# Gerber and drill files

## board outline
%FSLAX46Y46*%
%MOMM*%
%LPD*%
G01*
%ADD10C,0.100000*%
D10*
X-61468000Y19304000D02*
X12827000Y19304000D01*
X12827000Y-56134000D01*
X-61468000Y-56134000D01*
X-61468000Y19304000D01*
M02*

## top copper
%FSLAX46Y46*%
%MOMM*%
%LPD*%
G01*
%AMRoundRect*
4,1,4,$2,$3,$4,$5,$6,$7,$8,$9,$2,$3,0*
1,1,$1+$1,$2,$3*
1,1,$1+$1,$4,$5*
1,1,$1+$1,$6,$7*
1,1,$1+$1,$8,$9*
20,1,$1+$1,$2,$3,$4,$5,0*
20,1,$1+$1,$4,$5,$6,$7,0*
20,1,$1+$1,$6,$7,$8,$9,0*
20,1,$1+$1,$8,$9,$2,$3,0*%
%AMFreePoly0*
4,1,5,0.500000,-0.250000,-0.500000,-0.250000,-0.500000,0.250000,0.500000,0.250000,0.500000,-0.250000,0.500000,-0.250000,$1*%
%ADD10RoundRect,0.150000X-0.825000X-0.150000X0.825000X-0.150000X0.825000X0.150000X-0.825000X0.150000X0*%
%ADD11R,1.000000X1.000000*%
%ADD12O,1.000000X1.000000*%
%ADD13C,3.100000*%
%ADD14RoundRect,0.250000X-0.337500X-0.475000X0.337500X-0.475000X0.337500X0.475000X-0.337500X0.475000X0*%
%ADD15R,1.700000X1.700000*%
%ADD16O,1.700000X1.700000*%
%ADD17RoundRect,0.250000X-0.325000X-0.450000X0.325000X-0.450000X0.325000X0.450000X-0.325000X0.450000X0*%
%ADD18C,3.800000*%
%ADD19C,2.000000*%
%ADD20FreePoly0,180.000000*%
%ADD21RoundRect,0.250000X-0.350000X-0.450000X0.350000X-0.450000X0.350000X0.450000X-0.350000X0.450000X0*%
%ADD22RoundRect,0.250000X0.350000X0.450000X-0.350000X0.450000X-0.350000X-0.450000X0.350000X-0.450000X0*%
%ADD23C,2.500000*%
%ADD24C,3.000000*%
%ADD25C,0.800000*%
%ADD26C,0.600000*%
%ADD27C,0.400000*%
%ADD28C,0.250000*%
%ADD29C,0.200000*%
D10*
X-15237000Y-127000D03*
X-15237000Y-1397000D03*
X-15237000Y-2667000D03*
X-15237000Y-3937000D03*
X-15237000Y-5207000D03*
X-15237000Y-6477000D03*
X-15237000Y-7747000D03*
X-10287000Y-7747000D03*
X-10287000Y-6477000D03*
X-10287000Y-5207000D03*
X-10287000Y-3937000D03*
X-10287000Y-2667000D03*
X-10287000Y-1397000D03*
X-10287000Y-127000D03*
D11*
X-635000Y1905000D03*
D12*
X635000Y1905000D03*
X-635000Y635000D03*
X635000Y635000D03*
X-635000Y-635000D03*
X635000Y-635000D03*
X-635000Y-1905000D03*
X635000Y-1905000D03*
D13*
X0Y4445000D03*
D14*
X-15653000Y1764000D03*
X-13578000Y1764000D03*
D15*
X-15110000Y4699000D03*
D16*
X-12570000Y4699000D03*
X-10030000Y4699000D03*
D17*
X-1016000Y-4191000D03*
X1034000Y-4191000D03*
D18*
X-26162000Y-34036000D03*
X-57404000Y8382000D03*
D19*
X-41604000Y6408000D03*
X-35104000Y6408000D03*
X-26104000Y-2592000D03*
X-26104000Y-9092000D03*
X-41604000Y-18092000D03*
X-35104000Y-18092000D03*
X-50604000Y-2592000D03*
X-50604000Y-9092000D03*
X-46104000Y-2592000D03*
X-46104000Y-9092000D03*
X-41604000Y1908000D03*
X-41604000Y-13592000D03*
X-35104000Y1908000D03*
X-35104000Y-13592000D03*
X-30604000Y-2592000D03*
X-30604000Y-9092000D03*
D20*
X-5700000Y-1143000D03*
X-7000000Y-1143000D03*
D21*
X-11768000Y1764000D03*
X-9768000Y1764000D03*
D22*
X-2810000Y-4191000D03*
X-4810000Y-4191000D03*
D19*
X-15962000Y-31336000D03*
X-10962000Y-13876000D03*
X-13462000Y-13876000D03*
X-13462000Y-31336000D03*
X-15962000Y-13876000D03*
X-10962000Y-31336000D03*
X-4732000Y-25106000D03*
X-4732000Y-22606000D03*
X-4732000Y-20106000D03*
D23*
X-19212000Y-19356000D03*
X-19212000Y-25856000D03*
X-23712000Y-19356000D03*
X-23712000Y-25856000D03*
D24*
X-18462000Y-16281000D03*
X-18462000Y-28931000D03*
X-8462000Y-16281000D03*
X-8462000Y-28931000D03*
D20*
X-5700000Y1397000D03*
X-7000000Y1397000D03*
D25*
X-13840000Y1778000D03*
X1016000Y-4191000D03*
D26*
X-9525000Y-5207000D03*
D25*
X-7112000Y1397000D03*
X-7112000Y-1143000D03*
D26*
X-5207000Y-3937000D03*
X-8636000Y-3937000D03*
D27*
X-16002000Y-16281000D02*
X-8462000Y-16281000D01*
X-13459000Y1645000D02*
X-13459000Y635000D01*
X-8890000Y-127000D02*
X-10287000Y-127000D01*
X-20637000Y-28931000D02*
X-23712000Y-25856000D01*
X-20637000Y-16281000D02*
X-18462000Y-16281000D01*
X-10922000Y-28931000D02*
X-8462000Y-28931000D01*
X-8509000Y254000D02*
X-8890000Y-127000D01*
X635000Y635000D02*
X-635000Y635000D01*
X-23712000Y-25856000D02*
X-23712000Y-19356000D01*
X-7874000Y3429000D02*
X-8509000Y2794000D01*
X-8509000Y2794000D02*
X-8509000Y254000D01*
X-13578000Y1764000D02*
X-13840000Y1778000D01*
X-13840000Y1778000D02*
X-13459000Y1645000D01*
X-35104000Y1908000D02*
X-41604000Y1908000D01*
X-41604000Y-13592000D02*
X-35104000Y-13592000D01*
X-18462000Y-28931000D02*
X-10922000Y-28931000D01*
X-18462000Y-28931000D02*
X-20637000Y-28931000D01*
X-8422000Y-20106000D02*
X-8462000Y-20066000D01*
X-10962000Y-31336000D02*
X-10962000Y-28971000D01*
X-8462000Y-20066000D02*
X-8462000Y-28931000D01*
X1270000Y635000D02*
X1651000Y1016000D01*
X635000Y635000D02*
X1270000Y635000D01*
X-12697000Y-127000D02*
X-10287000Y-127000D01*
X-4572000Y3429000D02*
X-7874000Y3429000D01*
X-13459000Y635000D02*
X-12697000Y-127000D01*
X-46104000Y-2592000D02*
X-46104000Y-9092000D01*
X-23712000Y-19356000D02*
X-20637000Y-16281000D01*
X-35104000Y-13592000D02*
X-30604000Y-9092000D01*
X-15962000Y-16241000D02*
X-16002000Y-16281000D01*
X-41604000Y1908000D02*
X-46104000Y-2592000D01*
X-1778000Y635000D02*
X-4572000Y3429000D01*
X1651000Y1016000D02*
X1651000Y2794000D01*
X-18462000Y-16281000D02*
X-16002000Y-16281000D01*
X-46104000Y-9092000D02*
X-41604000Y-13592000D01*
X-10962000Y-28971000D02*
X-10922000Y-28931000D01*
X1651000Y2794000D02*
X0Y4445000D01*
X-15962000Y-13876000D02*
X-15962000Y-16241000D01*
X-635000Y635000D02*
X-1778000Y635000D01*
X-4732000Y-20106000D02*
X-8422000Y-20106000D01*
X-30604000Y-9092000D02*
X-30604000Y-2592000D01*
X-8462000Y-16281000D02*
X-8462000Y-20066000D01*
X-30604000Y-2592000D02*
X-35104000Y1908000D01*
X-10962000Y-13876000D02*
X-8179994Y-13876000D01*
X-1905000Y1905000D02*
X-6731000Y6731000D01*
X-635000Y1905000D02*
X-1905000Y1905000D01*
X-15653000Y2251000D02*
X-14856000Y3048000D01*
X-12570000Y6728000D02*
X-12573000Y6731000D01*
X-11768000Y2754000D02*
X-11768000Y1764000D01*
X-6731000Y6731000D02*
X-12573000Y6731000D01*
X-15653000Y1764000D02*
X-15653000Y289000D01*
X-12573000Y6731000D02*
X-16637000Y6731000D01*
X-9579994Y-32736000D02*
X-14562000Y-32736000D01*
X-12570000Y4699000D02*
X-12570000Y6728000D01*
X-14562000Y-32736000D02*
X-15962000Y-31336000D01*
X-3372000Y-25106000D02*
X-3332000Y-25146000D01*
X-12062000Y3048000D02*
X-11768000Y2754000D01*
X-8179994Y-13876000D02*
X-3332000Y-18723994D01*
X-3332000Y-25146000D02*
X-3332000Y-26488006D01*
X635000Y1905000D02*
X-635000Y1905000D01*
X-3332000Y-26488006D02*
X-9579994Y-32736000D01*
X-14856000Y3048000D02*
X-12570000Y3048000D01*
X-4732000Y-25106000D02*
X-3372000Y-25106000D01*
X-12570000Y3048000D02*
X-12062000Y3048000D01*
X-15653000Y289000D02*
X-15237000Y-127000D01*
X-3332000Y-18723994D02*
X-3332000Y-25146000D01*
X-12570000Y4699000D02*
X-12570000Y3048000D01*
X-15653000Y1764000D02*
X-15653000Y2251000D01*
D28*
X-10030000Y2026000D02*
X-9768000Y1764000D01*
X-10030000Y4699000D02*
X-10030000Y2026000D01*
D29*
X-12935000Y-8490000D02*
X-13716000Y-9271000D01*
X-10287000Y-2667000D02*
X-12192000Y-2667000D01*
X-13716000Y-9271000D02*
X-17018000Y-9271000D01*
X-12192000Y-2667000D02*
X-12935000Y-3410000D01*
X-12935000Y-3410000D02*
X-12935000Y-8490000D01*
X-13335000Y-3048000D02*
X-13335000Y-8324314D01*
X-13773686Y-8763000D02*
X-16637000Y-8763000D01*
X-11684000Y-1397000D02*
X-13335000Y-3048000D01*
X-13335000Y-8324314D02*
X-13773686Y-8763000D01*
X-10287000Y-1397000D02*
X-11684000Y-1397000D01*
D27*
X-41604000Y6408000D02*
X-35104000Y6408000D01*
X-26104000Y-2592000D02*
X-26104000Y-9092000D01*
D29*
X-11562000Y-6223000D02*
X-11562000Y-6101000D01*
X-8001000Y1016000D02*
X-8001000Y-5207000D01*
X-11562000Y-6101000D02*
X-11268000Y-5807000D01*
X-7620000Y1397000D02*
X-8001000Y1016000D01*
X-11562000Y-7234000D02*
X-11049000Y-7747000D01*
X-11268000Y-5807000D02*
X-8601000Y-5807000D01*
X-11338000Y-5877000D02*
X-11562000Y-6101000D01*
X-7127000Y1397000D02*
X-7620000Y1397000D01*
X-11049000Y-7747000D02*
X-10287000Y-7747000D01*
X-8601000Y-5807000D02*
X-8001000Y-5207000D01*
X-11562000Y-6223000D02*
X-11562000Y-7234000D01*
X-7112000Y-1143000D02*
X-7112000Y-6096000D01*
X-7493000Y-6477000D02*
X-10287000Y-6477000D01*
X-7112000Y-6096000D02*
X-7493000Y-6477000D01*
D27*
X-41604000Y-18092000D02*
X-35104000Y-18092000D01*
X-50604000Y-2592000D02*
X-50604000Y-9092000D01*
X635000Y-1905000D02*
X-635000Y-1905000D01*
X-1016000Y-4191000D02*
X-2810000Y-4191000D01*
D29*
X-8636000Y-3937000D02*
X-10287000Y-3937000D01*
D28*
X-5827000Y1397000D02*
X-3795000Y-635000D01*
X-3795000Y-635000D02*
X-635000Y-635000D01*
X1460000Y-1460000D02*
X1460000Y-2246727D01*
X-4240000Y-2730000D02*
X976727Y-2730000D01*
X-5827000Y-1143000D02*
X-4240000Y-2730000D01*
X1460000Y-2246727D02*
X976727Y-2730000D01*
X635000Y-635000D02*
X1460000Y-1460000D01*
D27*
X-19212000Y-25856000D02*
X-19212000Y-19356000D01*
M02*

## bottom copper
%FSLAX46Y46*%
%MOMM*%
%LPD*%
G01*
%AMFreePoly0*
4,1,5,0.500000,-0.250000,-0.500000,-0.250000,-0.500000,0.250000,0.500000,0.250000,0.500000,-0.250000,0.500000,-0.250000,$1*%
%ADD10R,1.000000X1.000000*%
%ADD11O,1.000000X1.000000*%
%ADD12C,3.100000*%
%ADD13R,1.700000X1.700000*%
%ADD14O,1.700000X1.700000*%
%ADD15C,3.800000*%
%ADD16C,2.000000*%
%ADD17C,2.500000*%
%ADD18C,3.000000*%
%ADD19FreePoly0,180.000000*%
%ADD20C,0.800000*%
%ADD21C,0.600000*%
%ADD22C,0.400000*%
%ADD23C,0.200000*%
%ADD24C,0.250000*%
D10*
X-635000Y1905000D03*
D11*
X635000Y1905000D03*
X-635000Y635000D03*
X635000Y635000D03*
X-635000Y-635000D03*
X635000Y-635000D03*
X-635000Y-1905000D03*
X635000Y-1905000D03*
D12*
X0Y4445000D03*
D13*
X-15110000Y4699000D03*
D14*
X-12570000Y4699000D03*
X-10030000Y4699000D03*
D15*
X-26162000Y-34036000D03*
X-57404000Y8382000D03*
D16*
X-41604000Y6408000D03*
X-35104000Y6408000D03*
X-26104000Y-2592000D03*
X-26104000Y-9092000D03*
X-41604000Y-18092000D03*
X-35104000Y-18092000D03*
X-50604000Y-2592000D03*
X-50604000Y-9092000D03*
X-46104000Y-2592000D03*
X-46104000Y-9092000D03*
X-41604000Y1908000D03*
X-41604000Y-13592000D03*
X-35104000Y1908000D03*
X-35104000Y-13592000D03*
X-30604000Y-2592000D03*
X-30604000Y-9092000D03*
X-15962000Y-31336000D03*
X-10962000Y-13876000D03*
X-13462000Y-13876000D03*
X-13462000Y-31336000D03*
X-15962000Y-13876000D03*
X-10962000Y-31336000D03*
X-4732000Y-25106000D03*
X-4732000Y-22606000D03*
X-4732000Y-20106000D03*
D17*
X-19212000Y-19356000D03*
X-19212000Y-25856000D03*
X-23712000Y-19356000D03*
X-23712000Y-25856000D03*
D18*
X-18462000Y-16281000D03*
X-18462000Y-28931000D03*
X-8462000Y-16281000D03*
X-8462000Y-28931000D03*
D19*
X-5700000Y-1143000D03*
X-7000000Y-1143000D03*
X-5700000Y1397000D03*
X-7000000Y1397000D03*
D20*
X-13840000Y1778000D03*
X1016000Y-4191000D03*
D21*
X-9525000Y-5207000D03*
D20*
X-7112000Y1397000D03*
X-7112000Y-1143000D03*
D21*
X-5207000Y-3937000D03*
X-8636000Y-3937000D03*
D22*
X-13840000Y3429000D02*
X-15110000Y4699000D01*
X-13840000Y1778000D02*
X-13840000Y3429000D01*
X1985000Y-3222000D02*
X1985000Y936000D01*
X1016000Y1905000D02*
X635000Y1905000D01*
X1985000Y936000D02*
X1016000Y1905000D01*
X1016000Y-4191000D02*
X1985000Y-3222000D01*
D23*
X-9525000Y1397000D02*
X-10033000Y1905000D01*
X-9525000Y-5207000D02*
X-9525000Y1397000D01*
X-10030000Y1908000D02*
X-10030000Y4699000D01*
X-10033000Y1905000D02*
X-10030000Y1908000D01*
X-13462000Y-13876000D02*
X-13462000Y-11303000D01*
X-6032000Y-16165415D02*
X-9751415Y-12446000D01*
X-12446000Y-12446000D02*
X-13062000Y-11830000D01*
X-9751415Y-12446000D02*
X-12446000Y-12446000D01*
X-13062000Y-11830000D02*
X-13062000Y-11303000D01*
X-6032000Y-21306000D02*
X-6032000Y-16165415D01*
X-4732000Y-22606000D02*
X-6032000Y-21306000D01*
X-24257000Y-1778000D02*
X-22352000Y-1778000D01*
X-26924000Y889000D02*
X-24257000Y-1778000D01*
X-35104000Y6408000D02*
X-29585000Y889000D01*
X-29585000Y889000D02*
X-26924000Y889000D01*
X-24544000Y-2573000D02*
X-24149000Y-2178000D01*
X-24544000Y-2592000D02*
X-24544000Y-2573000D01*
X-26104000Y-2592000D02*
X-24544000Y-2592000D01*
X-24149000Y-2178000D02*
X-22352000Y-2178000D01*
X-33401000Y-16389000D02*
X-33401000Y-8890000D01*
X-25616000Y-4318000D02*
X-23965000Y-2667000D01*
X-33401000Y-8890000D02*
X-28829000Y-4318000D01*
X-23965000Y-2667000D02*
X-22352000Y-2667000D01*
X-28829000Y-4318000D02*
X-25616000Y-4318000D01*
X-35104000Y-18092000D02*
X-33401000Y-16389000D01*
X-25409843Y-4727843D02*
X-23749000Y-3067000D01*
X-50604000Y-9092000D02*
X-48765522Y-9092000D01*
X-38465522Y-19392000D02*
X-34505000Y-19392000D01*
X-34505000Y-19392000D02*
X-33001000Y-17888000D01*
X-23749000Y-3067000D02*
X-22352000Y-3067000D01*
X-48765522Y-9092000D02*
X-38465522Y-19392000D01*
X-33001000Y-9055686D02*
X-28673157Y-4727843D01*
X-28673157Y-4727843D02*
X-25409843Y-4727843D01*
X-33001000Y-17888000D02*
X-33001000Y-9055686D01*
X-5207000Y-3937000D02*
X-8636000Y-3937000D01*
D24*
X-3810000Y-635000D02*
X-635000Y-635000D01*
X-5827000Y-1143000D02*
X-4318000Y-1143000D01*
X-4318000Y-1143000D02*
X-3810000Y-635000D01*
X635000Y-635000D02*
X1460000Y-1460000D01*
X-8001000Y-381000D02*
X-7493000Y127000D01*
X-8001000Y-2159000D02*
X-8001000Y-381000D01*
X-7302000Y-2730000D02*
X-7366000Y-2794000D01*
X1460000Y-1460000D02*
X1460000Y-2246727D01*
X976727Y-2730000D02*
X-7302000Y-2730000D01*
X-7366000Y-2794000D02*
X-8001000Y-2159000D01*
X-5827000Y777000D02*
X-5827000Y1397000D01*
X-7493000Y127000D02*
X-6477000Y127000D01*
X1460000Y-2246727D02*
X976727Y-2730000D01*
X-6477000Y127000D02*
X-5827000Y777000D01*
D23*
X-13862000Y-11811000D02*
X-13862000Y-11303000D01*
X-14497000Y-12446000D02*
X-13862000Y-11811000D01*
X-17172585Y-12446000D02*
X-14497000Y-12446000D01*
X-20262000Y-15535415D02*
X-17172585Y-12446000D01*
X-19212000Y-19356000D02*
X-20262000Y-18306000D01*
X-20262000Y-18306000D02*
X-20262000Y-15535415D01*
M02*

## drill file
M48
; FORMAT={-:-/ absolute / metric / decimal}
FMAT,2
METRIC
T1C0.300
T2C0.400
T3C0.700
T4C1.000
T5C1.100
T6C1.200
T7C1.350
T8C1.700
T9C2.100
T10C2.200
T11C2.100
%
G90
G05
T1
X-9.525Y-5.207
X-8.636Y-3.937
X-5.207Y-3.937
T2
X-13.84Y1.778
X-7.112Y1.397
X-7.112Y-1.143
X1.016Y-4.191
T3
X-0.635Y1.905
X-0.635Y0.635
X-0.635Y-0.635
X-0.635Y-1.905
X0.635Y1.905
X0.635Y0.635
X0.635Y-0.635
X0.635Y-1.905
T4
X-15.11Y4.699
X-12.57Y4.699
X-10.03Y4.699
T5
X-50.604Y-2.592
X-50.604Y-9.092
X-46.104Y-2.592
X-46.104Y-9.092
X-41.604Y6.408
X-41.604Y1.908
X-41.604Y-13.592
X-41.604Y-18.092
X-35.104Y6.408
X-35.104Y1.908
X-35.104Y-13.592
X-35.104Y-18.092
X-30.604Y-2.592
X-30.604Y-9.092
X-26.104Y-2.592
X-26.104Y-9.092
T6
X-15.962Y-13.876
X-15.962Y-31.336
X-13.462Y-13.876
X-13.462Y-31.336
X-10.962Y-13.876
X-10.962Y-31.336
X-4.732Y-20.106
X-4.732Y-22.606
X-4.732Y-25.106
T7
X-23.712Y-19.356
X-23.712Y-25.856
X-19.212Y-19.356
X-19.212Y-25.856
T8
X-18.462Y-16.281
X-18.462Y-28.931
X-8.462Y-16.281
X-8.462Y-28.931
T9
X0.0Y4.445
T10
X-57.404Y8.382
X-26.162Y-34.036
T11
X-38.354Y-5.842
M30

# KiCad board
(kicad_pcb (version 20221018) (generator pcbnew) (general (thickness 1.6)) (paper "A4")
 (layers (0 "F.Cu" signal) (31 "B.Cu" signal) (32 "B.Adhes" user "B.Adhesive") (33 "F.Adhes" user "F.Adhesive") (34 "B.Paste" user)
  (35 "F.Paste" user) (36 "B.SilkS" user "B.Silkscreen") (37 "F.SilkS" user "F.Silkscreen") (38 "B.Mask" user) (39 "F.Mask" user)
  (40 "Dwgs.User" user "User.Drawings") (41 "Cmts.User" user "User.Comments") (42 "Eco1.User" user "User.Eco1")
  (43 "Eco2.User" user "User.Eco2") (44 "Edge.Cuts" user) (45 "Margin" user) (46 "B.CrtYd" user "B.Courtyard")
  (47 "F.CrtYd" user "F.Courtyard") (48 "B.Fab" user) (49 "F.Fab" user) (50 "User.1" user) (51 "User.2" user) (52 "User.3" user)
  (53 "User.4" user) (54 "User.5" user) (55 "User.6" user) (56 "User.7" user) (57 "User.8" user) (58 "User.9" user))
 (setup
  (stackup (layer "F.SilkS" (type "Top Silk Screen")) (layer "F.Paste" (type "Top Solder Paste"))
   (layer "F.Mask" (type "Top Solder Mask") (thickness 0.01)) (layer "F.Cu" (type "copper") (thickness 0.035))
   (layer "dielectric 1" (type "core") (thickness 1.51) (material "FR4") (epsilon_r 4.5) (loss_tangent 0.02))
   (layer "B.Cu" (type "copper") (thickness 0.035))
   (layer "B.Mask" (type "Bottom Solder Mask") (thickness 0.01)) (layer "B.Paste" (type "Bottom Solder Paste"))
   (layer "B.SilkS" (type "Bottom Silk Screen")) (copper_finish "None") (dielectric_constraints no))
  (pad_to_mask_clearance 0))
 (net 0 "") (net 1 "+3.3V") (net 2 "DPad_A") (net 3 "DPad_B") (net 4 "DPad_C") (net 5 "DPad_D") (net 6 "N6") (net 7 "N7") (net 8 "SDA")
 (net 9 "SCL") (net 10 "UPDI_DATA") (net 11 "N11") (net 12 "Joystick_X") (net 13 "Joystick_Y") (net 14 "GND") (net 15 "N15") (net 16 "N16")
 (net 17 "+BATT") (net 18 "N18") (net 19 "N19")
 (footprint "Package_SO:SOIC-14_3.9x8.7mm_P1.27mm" (layer "F.Cu") (at -12.762 3.937)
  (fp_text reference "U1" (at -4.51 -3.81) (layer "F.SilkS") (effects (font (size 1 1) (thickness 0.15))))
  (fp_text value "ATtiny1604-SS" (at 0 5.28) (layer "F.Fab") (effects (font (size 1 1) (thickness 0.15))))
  (pad "1" smd roundrect (at -2.475 -3.81) (size 1.95 0.6) (layers "F.Cu" "F.Paste" "F.Mask") (roundrect_rratio 0.25) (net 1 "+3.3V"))
  (pad "2" smd roundrect (at -2.475 -2.54) (size 1.95 0.6) (layers "F.Cu" "F.Paste" "F.Mask") (roundrect_rratio 0.25) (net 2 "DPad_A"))
  (pad "3" smd roundrect (at -2.475 -1.27) (size 1.95 0.6) (layers "F.Cu" "F.Paste" "F.Mask") (roundrect_rratio 0.25) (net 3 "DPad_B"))
  (pad "4" smd roundrect (at -2.475 0) (size 1.95 0.6) (layers "F.Cu" "F.Paste" "F.Mask") (roundrect_rratio 0.25) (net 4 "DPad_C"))
  (pad "5" smd roundrect (at -2.475 1.27) (size 1.95 0.6) (layers "F.Cu" "F.Paste" "F.Mask") (roundrect_rratio 0.25) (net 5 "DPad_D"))
  (pad "6" smd roundrect (at -2.475 2.54) (size 1.95 0.6) (layers "F.Cu" "F.Paste" "F.Mask") (roundrect_rratio 0.25) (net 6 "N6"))
  (pad "7" smd roundrect (at -2.475 3.81) (size 1.95 0.6) (layers "F.Cu" "F.Paste" "F.Mask") (roundrect_rratio 0.25) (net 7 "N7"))
  (pad "8" smd roundrect (at 2.475 3.81) (size 1.95 0.6) (layers "F.Cu" "F.Paste" "F.Mask") (roundrect_rratio 0.25) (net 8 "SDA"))
  (pad "9" smd roundrect (at 2.475 2.54) (size 1.95 0.6) (layers "F.Cu" "F.Paste" "F.Mask") (roundrect_rratio 0.25) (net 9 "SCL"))
  (pad "10" smd roundrect (at 2.475 1.27) (size 1.95 0.6) (layers "F.Cu" "F.Paste" "F.Mask") (roundrect_rratio 0.25) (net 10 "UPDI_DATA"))
  (pad "11" smd roundrect (at 2.475 0) (size 1.95 0.6) (layers "F.Cu" "F.Paste" "F.Mask") (roundrect_rratio 0.25) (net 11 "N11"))
  (pad "12" smd roundrect (at 2.475 -1.27) (size 1.95 0.6) (layers "F.Cu" "F.Paste" "F.Mask") (roundrect_rratio 0.25) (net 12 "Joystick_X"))
  (pad "13" smd roundrect (at 2.475 -2.54) (size 1.95 0.6) (layers "F.Cu" "F.Paste" "F.Mask") (roundrect_rratio 0.25) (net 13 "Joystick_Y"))
  (pad "14" smd roundrect (at 2.475 -3.81) (size 1.95 0.6) (layers "F.Cu" "F.Paste" "F.Mask") (roundrect_rratio 0.25) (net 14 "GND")))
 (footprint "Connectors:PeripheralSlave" (layer "F.Cu") (at 0 0)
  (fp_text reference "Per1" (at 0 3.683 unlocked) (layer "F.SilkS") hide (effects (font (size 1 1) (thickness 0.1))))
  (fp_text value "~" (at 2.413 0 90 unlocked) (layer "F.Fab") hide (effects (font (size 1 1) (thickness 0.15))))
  (pad "1" thru_hole rect (at -0.635 -1.905) (size 1 1) (drill 0.7) (layers "*.Cu" "*.Mask") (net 1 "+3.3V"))
  (pad "2" thru_hole oval (at 0.635 -1.905) (size 1 1) (drill 0.7) (layers "*.Cu" "*.Mask") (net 1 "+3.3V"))
  (pad "3" thru_hole oval (at -0.635 -0.635) (size 1 1) (drill 0.7) (layers "*.Cu" "*.Mask") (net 14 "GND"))
  (pad "4" thru_hole oval (at 0.635 -0.635) (size 1 1) (drill 0.7) (layers "*.Cu" "*.Mask") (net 14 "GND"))
  (pad "5" thru_hole oval (at -0.635 0.635) (size 1 1) (drill 0.7) (layers "*.Cu" "*.Mask") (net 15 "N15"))
  (pad "6" thru_hole oval (at 0.635 0.635) (size 1 1) (drill 0.7) (layers "*.Cu" "*.Mask") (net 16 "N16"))
  (pad "7" thru_hole oval (at -0.635 1.905) (size 1 1) (drill 0.7) (layers "*.Cu" "*.Mask") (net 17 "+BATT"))
  (pad "8" thru_hole oval (at 0.635 1.905) (size 1 1) (drill 0.7) (layers "*.Cu" "*.Mask") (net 17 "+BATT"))
  (pad "9" thru_hole circle (at 0 -4.445) (size 3.1 3.1) (drill 2.1) (layers "*.Cu" "*.Mask") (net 14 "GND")))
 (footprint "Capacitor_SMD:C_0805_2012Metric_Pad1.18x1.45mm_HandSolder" (layer "F.Cu") (at -14.6155 -1.764)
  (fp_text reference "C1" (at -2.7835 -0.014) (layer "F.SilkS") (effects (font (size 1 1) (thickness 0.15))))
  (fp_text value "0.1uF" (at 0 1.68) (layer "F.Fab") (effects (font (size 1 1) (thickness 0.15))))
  (pad "1" smd roundrect (at -1.0375 0) (size 1.175 1.45) (layers "F.Cu" "F.Paste" "F.Mask") (roundrect_rratio 0.212766) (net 1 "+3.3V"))
  (pad "2" smd roundrect (at 1.0375 0) (size 1.175 1.45) (layers "F.Cu" "F.Paste" "F.Mask") (roundrect_rratio 0.212766) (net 14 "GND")))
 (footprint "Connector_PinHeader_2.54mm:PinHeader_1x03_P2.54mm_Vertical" (layer "F.Cu") (at -15.11 -4.699 90)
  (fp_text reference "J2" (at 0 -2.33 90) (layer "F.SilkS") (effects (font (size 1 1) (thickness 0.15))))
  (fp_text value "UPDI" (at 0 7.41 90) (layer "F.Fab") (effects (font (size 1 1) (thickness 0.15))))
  (pad "1" thru_hole rect (at 0 0 90) (size 1.7 1.7) (drill 1) (layers "*.Cu" "*.Mask") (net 14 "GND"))
  (pad "2" thru_hole oval (at 0 2.54 90) (size 1.7 1.7) (drill 1) (layers "*.Cu" "*.Mask") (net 1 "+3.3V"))
  (pad "3" thru_hole oval (at 0 5.08 90) (size 1.7 1.7) (drill 1) (layers "*.Cu" "*.Mask") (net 10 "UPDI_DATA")))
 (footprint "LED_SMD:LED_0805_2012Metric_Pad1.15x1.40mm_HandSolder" (layer "F.Cu") (at 0.009 4.191)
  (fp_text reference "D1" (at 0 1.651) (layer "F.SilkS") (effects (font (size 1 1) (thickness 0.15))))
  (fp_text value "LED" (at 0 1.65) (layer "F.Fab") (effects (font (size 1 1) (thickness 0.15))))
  (pad "1" smd roundrect (at -1.025 0) (size 1.15 1.4) (layers "F.Cu" "F.Paste" "F.Mask") (roundrect_rratio 0.217391) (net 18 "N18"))
  (pad "2" smd roundrect (at 1.025 0) (size 1.15 1.4) (layers "F.Cu" "F.Paste" "F.Mask") (roundrect_rratio 0.217391) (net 1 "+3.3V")))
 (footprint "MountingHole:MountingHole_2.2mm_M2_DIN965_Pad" (layer "F.Cu") (at -26.162 34.036)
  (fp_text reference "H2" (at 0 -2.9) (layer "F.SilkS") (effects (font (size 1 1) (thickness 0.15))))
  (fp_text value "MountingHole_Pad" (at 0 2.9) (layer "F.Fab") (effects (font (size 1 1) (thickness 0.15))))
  (pad "1" thru_hole circle (at 0 0) (size 3.8 3.8) (drill 2.2) (layers "*.Cu" "*.Mask") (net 14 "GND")))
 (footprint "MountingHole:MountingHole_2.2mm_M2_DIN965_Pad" (layer "F.Cu") (at -57.404 -8.382)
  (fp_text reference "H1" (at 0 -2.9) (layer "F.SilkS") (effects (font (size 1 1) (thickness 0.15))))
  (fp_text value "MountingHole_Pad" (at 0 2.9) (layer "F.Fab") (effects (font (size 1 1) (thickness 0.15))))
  (pad "1" thru_hole circle (at 0 0) (size 3.8 3.8) (drill 2.2) (layers "*.Cu" "*.Mask") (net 14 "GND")))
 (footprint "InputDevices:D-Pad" (layer "F.Cu") (at -38.354 5.842)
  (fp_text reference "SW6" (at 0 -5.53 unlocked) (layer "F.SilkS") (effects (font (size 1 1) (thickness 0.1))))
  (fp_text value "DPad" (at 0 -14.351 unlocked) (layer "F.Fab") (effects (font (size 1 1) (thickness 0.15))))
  (pad "" np_thru_hole circle (at 0 0 90) (size 2 2) (drill 2.1) (layers "F&B.Cu" "*.Mask"))
  (pad "1" thru_hole circle (at -3.25 -12.25 90) (size 2 2) (drill 1.1) (layers "*.Cu" "*.Mask") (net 2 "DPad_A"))
  (pad "1" thru_hole circle (at 3.25 -12.25 90) (size 2 2) (drill 1.1) (layers "*.Cu" "*.Mask") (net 2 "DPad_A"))
  (pad "2" thru_hole circle (at 12.25 -3.25) (size 2 2) (drill 1.1) (layers "*.Cu" "*.Mask") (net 3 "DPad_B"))
  (pad "2" thru_hole circle (at 12.25 3.25) (size 2 2) (drill 1.1) (layers "*.Cu" "*.Mask") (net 3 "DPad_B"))
  (pad "3" thru_hole circle (at -3.25 12.25 270) (size 2 2) (drill 1.1) (layers "*.Cu" "*.Mask") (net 4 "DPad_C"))
  (pad "3" thru_hole circle (at 3.25 12.25 270) (size 2 2) (drill 1.1) (layers "*.Cu" "*.Mask") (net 4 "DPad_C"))
  (pad "4" thru_hole circle (at -12.25 -3.25 180) (size 2 2) (drill 1.1) (layers "*.Cu" "*.Mask") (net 5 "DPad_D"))
  (pad "4" thru_hole circle (at -12.25 3.25 180) (size 2 2) (drill 1.1) (layers "*.Cu" "*.Mask") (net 5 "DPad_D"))
  (pad "5" thru_hole circle (at -7.75 -3.25 180) (size 2 2) (drill 1.1) (layers "*.Cu" "*.Mask") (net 14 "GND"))
  (pad "5" thru_hole circle (at -7.75 3.25 180) (size 2 2) (drill 1.1) (layers "*.Cu" "*.Mask") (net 14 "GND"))
  (pad "5" thru_hole circle (at -3.25 -7.75 90) (size 2 2) (drill 1.1) (layers "*.Cu" "*.Mask") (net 14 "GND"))
  (pad "5" thru_hole circle (at -3.25 7.75 270) (size 2 2) (drill 1.1) (layers "*.Cu" "*.Mask") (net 14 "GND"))
  (pad "5" thru_hole circle (at 3.25 -7.75 90) (size 2 2) (drill 1.1) (layers "*.Cu" "*.Mask") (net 14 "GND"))
  (pad "5" thru_hole circle (at 3.25 7.75 270) (size 2 2) (drill 1.1) (layers "*.Cu" "*.Mask") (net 14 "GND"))
  (pad "5" thru_hole circle (at 7.75 -3.25) (size 2 2) (drill 1.1) (layers "*.Cu" "*.Mask") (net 14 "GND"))
  (pad "5" thru_hole circle (at 7.75 3.25) (size 2 2) (drill 1.1) (layers "*.Cu" "*.Mask") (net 14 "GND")))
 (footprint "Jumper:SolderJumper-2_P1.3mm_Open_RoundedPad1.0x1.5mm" (layer "F.Cu") (at -6.35 1.143 180)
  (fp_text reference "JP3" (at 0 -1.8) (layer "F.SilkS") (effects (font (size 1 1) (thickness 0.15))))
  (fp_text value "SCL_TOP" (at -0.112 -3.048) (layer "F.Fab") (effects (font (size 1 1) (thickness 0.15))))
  (pad "1" smd custom (at -0.65 0 180) (size 1 0.5) (layers "F.Cu" "F.Mask") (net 16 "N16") (zone_connect 2) (thermal_bridge_angle 45)
   (options (clearance outline) (anchor rect)) (primitives))
  (pad "2" smd custom (at 0.65 0 180) (size 1 0.5) (layers "F.Cu" "F.Mask") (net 9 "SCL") (zone_connect 2) (thermal_bridge_angle 45)
   (options (clearance outline) (anchor rect)) (primitives)))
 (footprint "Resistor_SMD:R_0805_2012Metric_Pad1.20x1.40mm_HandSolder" (layer "F.Cu") (at -10.768 -1.764)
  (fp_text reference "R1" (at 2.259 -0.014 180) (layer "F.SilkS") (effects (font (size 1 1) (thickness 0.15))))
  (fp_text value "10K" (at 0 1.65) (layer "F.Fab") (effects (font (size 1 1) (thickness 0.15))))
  (pad "1" smd roundrect (at -1 0) (size 1.2 1.4) (layers "F.Cu" "F.Paste" "F.Mask") (roundrect_rratio 0.208333) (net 1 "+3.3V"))
  (pad "2" smd roundrect (at 1 0) (size 1.2 1.4) (layers "F.Cu" "F.Paste" "F.Mask") (roundrect_rratio 0.208333) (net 10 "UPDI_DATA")))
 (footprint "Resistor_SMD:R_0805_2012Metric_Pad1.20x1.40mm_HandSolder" (layer "F.Cu") (at -3.81 4.191 180)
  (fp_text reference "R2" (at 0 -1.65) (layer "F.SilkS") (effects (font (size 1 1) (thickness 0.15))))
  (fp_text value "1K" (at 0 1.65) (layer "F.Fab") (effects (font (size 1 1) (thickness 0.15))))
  (pad "1" smd roundrect (at -1 0 180) (size 1.2 1.4) (layers "F.Cu" "F.Paste" "F.Mask") (roundrect_rratio 0.208333) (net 18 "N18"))
  (pad "2" smd roundrect (at 1 0 180) (size 1.2 1.4) (layers "F.Cu" "F.Paste" "F.Mask") (roundrect_rratio 0.208333) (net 11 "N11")))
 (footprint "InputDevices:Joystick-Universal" (layer "F.Cu") (at -13.462 22.606)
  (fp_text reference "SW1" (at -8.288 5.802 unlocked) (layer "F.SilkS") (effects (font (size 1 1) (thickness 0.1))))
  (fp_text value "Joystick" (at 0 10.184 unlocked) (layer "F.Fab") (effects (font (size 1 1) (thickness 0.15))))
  (pad "1" thru_hole circle (at -2.5 8.73) (size 2 2) (drill 1.2) (layers "*.Cu" "*.Mask") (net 1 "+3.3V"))
  (pad "1" thru_hole circle (at 2.5 -8.73 180) (size 2 2) (drill 1.2) (layers "*.Cu" "*.Mask") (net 1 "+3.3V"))
  (pad "2" thru_hole circle (at 0 -8.73 180) (size 2 2) (drill 1.2) (layers "*.Cu" "*.Mask") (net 12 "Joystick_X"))
  (pad "2" thru_hole circle (at 0 8.73) (size 2 2) (drill 1.2) (layers "*.Cu" "*.Mask") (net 12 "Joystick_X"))
  (pad "3" thru_hole circle (at -2.5 -8.73 180) (size 2 2) (drill 1.2) (layers "*.Cu" "*.Mask") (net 14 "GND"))
  (pad "3" thru_hole circle (at 2.5 8.73) (size 2 2) (drill 1.2) (layers "*.Cu" "*.Mask") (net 14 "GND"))
  (pad "4" thru_hole circle (at 8.73 2.5 90) (size 2 2) (drill 1.2) (layers "*.Cu" "*.Mask") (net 1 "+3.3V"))
  (pad "5" thru_hole circle (at 8.73 0 90) (size 2 2) (drill 1.2) (layers "*.Cu" "*.Mask") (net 13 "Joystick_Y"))
  (pad "6" thru_hole circle (at 8.73 -2.5 90) (size 2 2) (drill 1.2) (layers "*.Cu" "*.Mask") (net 14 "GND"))
  (pad "7" thru_hole circle (at -5.75 -3.25) (size 2.5 2.5) (drill 1.35) (layers "*.Cu" "*.Mask") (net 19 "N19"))
  (pad "7" thru_hole circle (at -5.75 3.25) (size 2.5 2.5) (drill 1.35) (layers "*.Cu" "*.Mask") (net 19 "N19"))
  (pad "8" thru_hole circle (at -10.25 -3.25) (size 2.5 2.5) (drill 1.35) (layers "*.Cu" "*.Mask") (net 14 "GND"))
  (pad "8" thru_hole circle (at -10.25 3.25) (size 2.5 2.5) (drill 1.35) (layers "*.Cu" "*.Mask") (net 14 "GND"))
  (pad "9" thru_hole circle (at -5 -6.325 90) (size 3 3) (drill 1.7) (layers "*.Cu" "*.Mask") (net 14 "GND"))
  (pad "9" thru_hole circle (at -5 6.325 180) (size 3 3) (drill 1.7) (layers "*.Cu" "*.Mask") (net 14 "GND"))
  (pad "9" thru_hole circle (at 5 -6.325 180) (size 3 3) (drill 1.7) (layers "*.Cu" "*.Mask") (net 14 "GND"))
  (pad "9" thru_hole circle (at 5 6.325 90) (size 3 3) (drill 1.7) (layers "*.Cu" "*.Mask") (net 14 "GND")))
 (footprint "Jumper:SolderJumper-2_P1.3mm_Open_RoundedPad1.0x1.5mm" (layer "F.Cu") (at -6.35 -1.397 180)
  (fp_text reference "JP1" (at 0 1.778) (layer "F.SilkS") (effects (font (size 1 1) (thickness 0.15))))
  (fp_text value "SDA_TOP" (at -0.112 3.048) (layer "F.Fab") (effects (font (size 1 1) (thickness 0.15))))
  (pad "1" smd custom (at -0.65 0 180) (size 1 0.5) (layers "F.Cu" "F.Mask") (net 15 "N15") (zone_connect 2) (thermal_bridge_angle 45)
   (options (clearance outline) (anchor rect)) (primitives))
  (pad "2" smd custom (at 0.65 0 180) (size 1 0.5) (layers "F.Cu" "F.Mask") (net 8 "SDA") (zone_connect 2) (thermal_bridge_angle 45)
   (options (clearance outline) (anchor rect)) (primitives)))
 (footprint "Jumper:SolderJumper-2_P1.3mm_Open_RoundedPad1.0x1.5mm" (layer "B.Cu") (at -6.35 1.143 180)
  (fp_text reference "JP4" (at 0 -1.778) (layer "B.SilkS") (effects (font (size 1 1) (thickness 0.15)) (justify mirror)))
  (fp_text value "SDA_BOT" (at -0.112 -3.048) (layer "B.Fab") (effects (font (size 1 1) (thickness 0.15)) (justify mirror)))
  (pad "1" smd custom (at -0.65 0 180) (size 1 0.5) (layers "B.Cu" "B.Mask") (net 15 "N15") (zone_connect 2) (thermal_bridge_angle 45)
   (options (clearance outline) (anchor rect)) (primitives))
  (pad "2" smd custom (at 0.65 0 180) (size 1 0.5) (layers "B.Cu" "B.Mask") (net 9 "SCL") (zone_connect 2) (thermal_bridge_angle 45)
   (options (clearance outline) (anchor rect)) (primitives)))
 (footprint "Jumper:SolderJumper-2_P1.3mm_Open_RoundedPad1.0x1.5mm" (layer "B.Cu") (at -6.35 -1.397 180)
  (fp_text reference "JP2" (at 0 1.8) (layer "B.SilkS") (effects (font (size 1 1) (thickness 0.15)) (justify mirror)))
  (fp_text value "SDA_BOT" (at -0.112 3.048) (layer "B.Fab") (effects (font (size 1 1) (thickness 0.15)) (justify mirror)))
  (pad "1" smd custom (at -0.65 0 180) (size 1 0.5) (layers "B.Cu" "B.Mask") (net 16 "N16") (zone_connect 2) (thermal_bridge_angle 45)
   (options (clearance outline) (anchor rect)) (primitives))
  (pad "2" smd custom (at 0.65 0 180) (size 1 0.5) (layers "B.Cu" "B.Mask") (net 8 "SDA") (zone_connect 2) (thermal_bridge_angle 45)
   (options (clearance outline) (anchor rect)) (primitives)))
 (gr_rect (start -61.468 -19.304) (end 12.827 56.134) (stroke (width 0.1) (type default)) (fill none) (layer "Edge.Cuts"))
 (segment (start -16.002 16.281) (end -8.462 16.281) (width 0.4) (layer "F.Cu") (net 14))
 (segment (start -13.459 -1.645) (end -13.459 -0.635) (width 0.4) (layer "F.Cu") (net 14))
 (segment (start -8.89 0.127) (end -10.287 0.127) (width 0.4) (layer "F.Cu") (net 14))
 (segment (start -20.637 28.931) (end -23.712 25.856) (width 0.4) (layer "F.Cu") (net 14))
 (segment (start -20.637 16.281) (end -18.462 16.281) (width 0.4) (layer "F.Cu") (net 14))
 (segment (start -10.922 28.931) (end -8.462 28.931) (width 0.4) (layer "F.Cu") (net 14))
 (segment (start -8.509 -0.254) (end -8.89 0.127) (width 0.4) (layer "F.Cu") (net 14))
 (segment (start 0.635 -0.635) (end -0.635 -0.635) (width 0.4) (layer "F.Cu") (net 14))
 (segment (start -23.712 25.856) (end -23.712 19.356) (width 0.4) (layer "F.Cu") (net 14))
 (segment (start -7.874 -3.429) (end -8.509 -2.794) (width 0.4) (layer "F.Cu") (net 14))
 (segment (start -8.509 -2.794) (end -8.509 -0.254) (width 0.4) (layer "F.Cu") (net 14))
 (segment (start -13.578 -1.764) (end -13.84 -1.778) (width 0.4) (layer "F.Cu") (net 14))
 (segment (start -13.84 -1.778) (end -13.459 -1.645) (width 0.4) (layer "F.Cu") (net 14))
 (segment (start -35.104 -1.908) (end -41.604 -1.908) (width 0.4) (layer "F.Cu") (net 14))
 (segment (start -41.604 13.592) (end -35.104 13.592) (width 0.4) (layer "F.Cu") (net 14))
 (segment (start -18.462 28.931) (end -10.922 28.931) (width 0.4) (layer "F.Cu") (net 14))
 (segment (start -18.462 28.931) (end -20.637 28.931) (width 0.4) (layer "F.Cu") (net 14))
 (segment (start -8.422 20.106) (end -8.462 20.066) (width 0.4) (layer "F.Cu") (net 14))
 (segment (start -10.962 31.336) (end -10.962 28.971) (width 0.4) (layer "F.Cu") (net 14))
 (segment (start -8.462 20.066) (end -8.462 28.931) (width 0.4) (layer "F.Cu") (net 14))
 (segment (start 1.27 -0.635) (end 1.651 -1.016) (width 0.4) (layer "F.Cu") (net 14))
 (segment (start 0.635 -0.635) (end 1.27 -0.635) (width 0.4) (layer "F.Cu") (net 14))
 (segment (start -12.697 0.127) (end -10.287 0.127) (width 0.4) (layer "F.Cu") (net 14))
 (segment (start -4.572 -3.429) (end -7.874 -3.429) (width 0.4) (layer "F.Cu") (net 14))
 (segment (start -13.459 -0.635) (end -12.697 0.127) (width 0.4) (layer "F.Cu") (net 14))
 (segment (start -46.104 2.592) (end -46.104 9.092) (width 0.4) (layer "F.Cu") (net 14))
 (segment (start -23.712 19.356) (end -20.637 16.281) (width 0.4) (layer "F.Cu") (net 14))
 (segment (start -35.104 13.592) (end -30.604 9.092) (width 0.4) (layer "F.Cu") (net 14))
 (segment (start -15.962 16.241) (end -16.002 16.281) (width 0.4) (layer "F.Cu") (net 14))
 (segment (start -41.604 -1.908) (end -46.104 2.592) (width 0.4) (layer "F.Cu") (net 14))
 (segment (start -1.778 -0.635) (end -4.572 -3.429) (width 0.4) (layer "F.Cu") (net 14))
 (segment (start 1.651 -1.016) (end 1.651 -2.794) (width 0.4) (layer "F.Cu") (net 14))
 (segment (start -18.462 16.281) (end -16.002 16.281) (width 0.4) (layer "F.Cu") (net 14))
 (segment (start -46.104 9.092) (end -41.604 13.592) (width 0.4) (layer "F.Cu") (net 14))
 (segment (start -10.962 28.971) (end -10.922 28.931) (width 0.4) (layer "F.Cu") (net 14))
 (segment (start 1.651 -2.794) (end 0 -4.445) (width 0.4) (layer "F.Cu") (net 14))
 (segment (start -15.962 13.876) (end -15.962 16.241) (width 0.4) (layer "F.Cu") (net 14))
 (segment (start -0.635 -0.635) (end -1.778 -0.635) (width 0.4) (layer "F.Cu") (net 14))
 (segment (start -4.732 20.106) (end -8.422 20.106) (width 0.4) (layer "F.Cu") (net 14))
 (segment (start -30.604 9.092) (end -30.604 2.592) (width 0.4) (layer "F.Cu") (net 14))
 (segment (start -8.462 16.281) (end -8.462 20.066) (width 0.4) (layer "F.Cu") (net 14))
 (segment (start -30.604 2.592) (end -35.104 -1.908) (width 0.4) (layer "F.Cu") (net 14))
 (via (at -13.84 -1.778) (size 0.8) (drill 0.4) (layers "F.Cu" "B.Cu") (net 14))
 (segment (start -13.84 -3.429) (end -15.11 -4.699) (width 0.4) (layer "B.Cu") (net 14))
 (segment (start -13.84 -1.778) (end -13.84 -3.429) (width 0.4) (layer "B.Cu") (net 14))
 (segment (start -10.962 13.876) (end -8.179994 13.876) (width 0.4) (layer "F.Cu") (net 1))
 (segment (start -1.905 -1.905) (end -6.731 -6.731) (width 0.4) (layer "F.Cu") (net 1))
 (segment (start -0.635 -1.905) (end -1.905 -1.905) (width 0.4) (layer "F.Cu") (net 1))
 (segment (start -15.653 -2.251) (end -14.856 -3.048) (width 0.4) (layer "F.Cu") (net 1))
 (segment (start -12.57 -6.728) (end -12.573 -6.731) (width 0.4) (layer "F.Cu") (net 1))
 (segment (start -11.768 -2.754) (end -11.768 -1.764) (width 0.4) (layer "F.Cu") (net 1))
 (segment (start -6.731 -6.731) (end -12.573 -6.731) (width 0.4) (layer "F.Cu") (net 1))
 (segment (start -15.653 -1.764) (end -15.653 -0.289) (width 0.4) (layer "F.Cu") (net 1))
 (segment (start -12.573 -6.731) (end -16.637 -6.731) (width 0.4) (layer "F.Cu") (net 1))
 (segment (start -9.579994 32.736) (end -14.562 32.736) (width 0.4) (layer "F.Cu") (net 1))
 (segment (start -12.57 -4.699) (end -12.57 -6.728) (width 0.4) (layer "F.Cu") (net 1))
 (segment (start -14.562 32.736) (end -15.962 31.336) (width 0.4) (layer "F.Cu") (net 1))
 (segment (start -3.372 25.106) (end -3.332 25.146) (width 0.4) (layer "F.Cu") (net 1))
 (segment (start -12.062 -3.048) (end -11.768 -2.754) (width 0.4) (layer "F.Cu") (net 1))
 (segment (start -8.179994 13.876) (end -3.332 18.723994) (width 0.4) (layer "F.Cu") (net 1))
 (segment (start -3.332 25.146) (end -3.332 26.488006) (width 0.4) (layer "F.Cu") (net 1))
 (segment (start 0.635 -1.905) (end -0.635 -1.905) (width 0.4) (layer "F.Cu") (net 1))
 (segment (start -3.332 26.488006) (end -9.579994 32.736) (width 0.4) (layer "F.Cu") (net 1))
 (segment (start -14.856 -3.048) (end -12.57 -3.048) (width 0.4) (layer "F.Cu") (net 1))
 (segment (start -4.732 25.106) (end -3.372 25.106) (width 0.4) (layer "F.Cu") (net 1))
 (segment (start -12.57 -3.048) (end -12.062 -3.048) (width 0.4) (layer "F.Cu") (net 1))
 (segment (start -15.653 -0.289) (end -15.237 0.127) (width 0.4) (layer "F.Cu") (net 1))
 (segment (start -3.332 18.723994) (end -3.332 25.146) (width 0.4) (layer "F.Cu") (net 1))
 (segment (start -12.57 -4.699) (end -12.57 -3.048) (width 0.4) (layer "F.Cu") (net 1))
 (segment (start -15.653 -1.764) (end -15.653 -2.251) (width 0.4) (layer "F.Cu") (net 1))
 (via (at 1.016 4.191) (size 0.8) (drill 0.4) (layers "F.Cu" "B.Cu") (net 1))
 (segment (start 1.985 3.222) (end 1.985 -0.936) (width 0.4) (layer "B.Cu") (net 1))
 (segment (start 1.016 -1.905) (end 0.635 -1.905) (width 0.4) (layer "B.Cu") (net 1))
 (segment (start 1.985 -0.936) (end 1.016 -1.905) (width 0.4) (layer "B.Cu") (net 1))
 (segment (start 1.016 4.191) (end 1.985 3.222) (width 0.4) (layer "B.Cu") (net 1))
 (segment (start -10.03 -2.026) (end -9.768 -1.764) (width 0.25) (layer "F.Cu") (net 10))
 (segment (start -10.03 -4.699) (end -10.03 -2.026) (width 0.25) (layer "F.Cu") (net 10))
 (via (at -9.525 5.207) (size 0.6) (drill 0.3) (layers "F.Cu" "B.Cu") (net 10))
 (segment (start -9.525 -1.397) (end -10.033 -1.905) (width 0.2) (layer "B.Cu") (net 10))
 (segment (start -9.525 5.207) (end -9.525 -1.397) (width 0.2) (layer "B.Cu") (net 10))
 (segment (start -10.03 -1.908) (end -10.03 -4.699) (width 0.2) (layer "B.Cu") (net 10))
 (segment (start -10.033 -1.905) (end -10.03 -1.908) (width 0.2) (layer "B.Cu") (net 10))
 (segment (start -12.935 8.49) (end -13.716 9.271) (width 0.2) (layer "F.Cu") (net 12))
 (segment (start -10.287 2.667) (end -12.192 2.667) (width 0.2) (layer "F.Cu") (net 12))
 (segment (start -13.716 9.271) (end -17.018 9.271) (width 0.2) (layer "F.Cu") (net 12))
 (segment (start -12.192 2.667) (end -12.935 3.41) (width 0.2) (layer "F.Cu") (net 12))
 (segment (start -12.935 3.41) (end -12.935 8.49) (width 0.2) (layer "F.Cu") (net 12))
 (segment (start -13.462 13.876) (end -13.462 11.303) (width 0.2) (layer "B.Cu") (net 12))
 (segment (start -13.335 3.048) (end -13.335 8.324314) (width 0.2) (layer "F.Cu") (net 13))
 (segment (start -13.773686 8.763) (end -16.637 8.763) (width 0.2) (layer "F.Cu") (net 13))
 (segment (start -11.684 1.397) (end -13.335 3.048) (width 0.2) (layer "F.Cu") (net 13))
 (segment (start -13.335 8.324314) (end -13.773686 8.763) (width 0.2) (layer "F.Cu") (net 13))
 (segment (start -10.287 1.397) (end -11.684 1.397) (width 0.2) (layer "F.Cu") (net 13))
 (segment (start -6.032 16.165415) (end -9.751415 12.446) (width 0.2) (layer "B.Cu") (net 13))
 (segment (start -12.446 12.446) (end -13.062 11.83) (width 0.2) (layer "B.Cu") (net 13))
 (segment (start -9.751415 12.446) (end -12.446 12.446) (width 0.2) (layer "B.Cu") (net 13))
 (segment (start -13.062 11.83) (end -13.062 11.303) (width 0.2) (layer "B.Cu") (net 13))
 (segment (start -6.032 21.306) (end -6.032 16.165415) (width 0.2) (layer "B.Cu") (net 13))
 (segment (start -4.732 22.606) (end -6.032 21.306) (width 0.2) (layer "B.Cu") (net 13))
 (segment (start -41.604 -6.408) (end -35.104 -6.408) (width 0.4) (layer "F.Cu") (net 2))
 (segment (start -24.257 1.778) (end -22.352 1.778) (width 0.2) (layer "B.Cu") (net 2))
 (segment (start -26.924 -0.889) (end -24.257 1.778) (width 0.2) (layer "B.Cu") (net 2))
 (segment (start -35.104 -6.408) (end -29.585 -0.889) (width 0.2) (layer "B.Cu") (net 2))
 (segment (start -29.585 -0.889) (end -26.924 -0.889) (width 0.2) (layer "B.Cu") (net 2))
 (segment (start -26.104 2.592) (end -26.104 9.092) (width 0.4) (layer "F.Cu") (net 3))
 (segment (start -24.544 2.573) (end -24.149 2.178) (width 0.2) (layer "B.Cu") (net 3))
 (segment (start -24.544 2.592) (end -24.544 2.573) (width 0.2) (layer "B.Cu") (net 3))
 (segment (start -26.104 2.592) (end -24.544 2.592) (width 0.2) (layer "B.Cu") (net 3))
 (segment (start -24.149 2.178) (end -22.352 2.178) (width 0.2) (layer "B.Cu") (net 3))
 (segment (start -11.562 6.223) (end -11.562 6.101) (width 0.2) (layer "F.Cu") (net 8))
 (segment (start -8.001 -1.016) (end -8.001 5.207) (width 0.2) (layer "F.Cu") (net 8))
 (segment (start -11.562 6.101) (end -11.268 5.807) (width 0.2) (layer "F.Cu") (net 8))
 (segment (start -7.62 -1.397) (end -8.001 -1.016) (width 0.2) (layer "F.Cu") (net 8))
 (segment (start -11.562 7.234) (end -11.049 7.747) (width 0.2) (layer "F.Cu") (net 8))
 (segment (start -11.268 5.807) (end -8.601 5.807) (width 0.2) (layer "F.Cu") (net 8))
 (segment (start -11.338 5.877) (end -11.562 6.101) (width 0.2) (layer "F.Cu") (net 8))
 (segment (start -7.127 -1.397) (end -7.62 -1.397) (width 0.2) (layer "F.Cu") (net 8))
 (segment (start -11.049 7.747) (end -10.287 7.747) (width 0.2) (layer "F.Cu") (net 8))
 (segment (start -8.601 5.807) (end -8.001 5.207) (width 0.2) (layer "F.Cu") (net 8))
 (segment (start -11.562 6.223) (end -11.562 7.234) (width 0.2) (layer "F.Cu") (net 8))
 (via (at -7.112 -1.397) (size 0.8) (drill 0.4) (layers "F.Cu" "B.Cu") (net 8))
 (segment (start -7.112 1.143) (end -7.112 6.096) (width 0.2) (layer "F.Cu") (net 9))
 (segment (start -7.493 6.477) (end -10.287 6.477) (width 0.2) (layer "F.Cu") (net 9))
 (segment (start -7.112 6.096) (end -7.493 6.477) (width 0.2) (layer "F.Cu") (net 9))
 (via (at -7.112 1.143) (size 0.8) (drill 0.4) (layers "F.Cu" "B.Cu") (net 9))
 (segment (start -41.604 18.092) (end -35.104 18.092) (width 0.4) (layer "F.Cu") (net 4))
 (segment (start -33.401 16.389) (end -33.401 8.89) (width 0.2) (layer "B.Cu") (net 4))
 (segment (start -25.616 4.318) (end -23.965 2.667) (width 0.2) (layer "B.Cu") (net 4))
 (segment (start -33.401 8.89) (end -28.829 4.318) (width 0.2) (layer "B.Cu") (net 4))
 (segment (start -23.965 2.667) (end -22.352 2.667) (width 0.2) (layer "B.Cu") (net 4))
 (segment (start -28.829 4.318) (end -25.616 4.318) (width 0.2) (layer "B.Cu") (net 4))
 (segment (start -35.104 18.092) (end -33.401 16.389) (width 0.2) (layer "B.Cu") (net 4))
 (segment (start -50.604 2.592) (end -50.604 9.092) (width 0.4) (layer "F.Cu") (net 5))
 (segment (start -25.409843 4.727843) (end -23.749 3.067) (width 0.2) (layer "B.Cu") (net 5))
 (segment (start -50.604 9.092) (end -48.765522 9.092) (width 0.2) (layer "B.Cu") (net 5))
 (segment (start -38.465522 19.392) (end -34.505 19.392) (width 0.2) (layer "B.Cu") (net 5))
 (segment (start -34.505 19.392) (end -33.001 17.888) (width 0.2) (layer "B.Cu") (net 5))
 (segment (start -23.749 3.067) (end -22.352 3.067) (width 0.2) (layer "B.Cu") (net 5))
 (segment (start -48.765522 9.092) (end -38.465522 19.392) (width 0.2) (layer "B.Cu") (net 5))
 (segment (start -33.001 9.055686) (end -28.673157 4.727843) (width 0.2) (layer "B.Cu") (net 5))
 (segment (start -28.673157 4.727843) (end -25.409843 4.727843) (width 0.2) (layer "B.Cu") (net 5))
 (segment (start -33.001 17.888) (end -33.001 9.055686) (width 0.2) (layer "B.Cu") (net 5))
 (segment (start 0.635 1.905) (end -0.635 1.905) (width 0.4) (layer "F.Cu") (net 17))
 (segment (start -1.016 4.191) (end -2.81 4.191) (width 0.4) (layer "F.Cu") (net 18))
 (segment (start -8.636 3.937) (end -10.287 3.937) (width 0.2) (layer "F.Cu") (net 11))
 (via (at -5.207 3.937) (size 0.6) (drill 0.3) (layers "F.Cu" "B.Cu") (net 11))
 (via (at -8.636 3.937) (size 0.6) (drill 0.3) (layers "F.Cu" "B.Cu") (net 11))
 (segment (start -5.207 3.937) (end -8.636 3.937) (width 0.2) (layer "B.Cu") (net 11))
 (segment (start -5.827 -1.397) (end -3.795 0.635) (width 0.25) (layer "F.Cu") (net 15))
 (segment (start -3.795 0.635) (end -0.635 0.635) (width 0.25) (layer "F.Cu") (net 15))
 (segment (start -3.81 0.635) (end -0.635 0.635) (width 0.25) (layer "B.Cu") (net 15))
 (segment (start -5.827 1.143) (end -4.318 1.143) (width 0.25) (layer "B.Cu") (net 15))
 (segment (start -4.318 1.143) (end -3.81 0.635) (width 0.25) (layer "B.Cu") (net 15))
 (segment (start 1.46 1.46) (end 1.46 2.246727) (width 0.25) (layer "F.Cu") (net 16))
 (segment (start -4.24 2.73) (end 0.976727 2.73) (width 0.25) (layer "F.Cu") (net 16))
 (segment (start -5.827 1.143) (end -4.24 2.73) (width 0.25) (layer "F.Cu") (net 16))
 (segment (start 1.46 2.246727) (end 0.976727 2.73) (width 0.25) (layer "F.Cu") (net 16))
 (segment (start 0.635 0.635) (end 1.46 1.46) (width 0.25) (layer "F.Cu") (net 16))
 (segment (start 0.635 0.635) (end 1.46 1.46) (width 0.25) (layer "B.Cu") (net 16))
 (segment (start -8.001 0.381) (end -7.493 -0.127) (width 0.25) (layer "B.Cu") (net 16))
 (segment (start -8.001 2.159) (end -8.001 0.381) (width 0.25) (layer "B.Cu") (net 16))
 (segment (start -7.302 2.73) (end -7.366 2.794) (width 0.25) (layer "B.Cu") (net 16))
 (segment (start 1.46 1.46) (end 1.46 2.246727) (width 0.25) (layer "B.Cu") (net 16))
 (segment (start 0.976727 2.73) (end -7.302 2.73) (width 0.25) (layer "B.Cu") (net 16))
 (segment (start -7.366 2.794) (end -8.001 2.159) (width 0.25) (layer "B.Cu") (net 16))
 (segment (start -5.827 -0.777) (end -5.827 -1.397) (width 0.25) (layer "B.Cu") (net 16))
 (segment (start -7.493 -0.127) (end -6.477 -0.127) (width 0.25) (layer "B.Cu") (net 16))
 (segment (start 1.46 2.246727) (end 0.976727 2.73) (width 0.25) (layer "B.Cu") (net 16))
 (segment (start -6.477 -0.127) (end -5.827 -0.777) (width 0.25) (layer "B.Cu") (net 16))
 (segment (start -19.212 25.856) (end -19.212 19.356) (width 0.4) (layer "F.Cu") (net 19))
 (segment (start -13.862 11.811) (end -13.862 11.303) (width 0.2) (layer "B.Cu") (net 19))
 (segment (start -14.497 12.446) (end -13.862 11.811) (width 0.2) (layer "B.Cu") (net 19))
 (segment (start -17.172585 12.446) (end -14.497 12.446) (width 0.2) (layer "B.Cu") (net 19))
 (segment (start -20.262 15.535415) (end -17.172585 12.446) (width 0.2) (layer "B.Cu") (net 19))
 (segment (start -19.212 19.356) (end -20.262 18.306) (width 0.2) (layer "B.Cu") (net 19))
 (segment (start -20.262 18.306) (end -20.262 15.535415) (width 0.2) (layer "B.Cu") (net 19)))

